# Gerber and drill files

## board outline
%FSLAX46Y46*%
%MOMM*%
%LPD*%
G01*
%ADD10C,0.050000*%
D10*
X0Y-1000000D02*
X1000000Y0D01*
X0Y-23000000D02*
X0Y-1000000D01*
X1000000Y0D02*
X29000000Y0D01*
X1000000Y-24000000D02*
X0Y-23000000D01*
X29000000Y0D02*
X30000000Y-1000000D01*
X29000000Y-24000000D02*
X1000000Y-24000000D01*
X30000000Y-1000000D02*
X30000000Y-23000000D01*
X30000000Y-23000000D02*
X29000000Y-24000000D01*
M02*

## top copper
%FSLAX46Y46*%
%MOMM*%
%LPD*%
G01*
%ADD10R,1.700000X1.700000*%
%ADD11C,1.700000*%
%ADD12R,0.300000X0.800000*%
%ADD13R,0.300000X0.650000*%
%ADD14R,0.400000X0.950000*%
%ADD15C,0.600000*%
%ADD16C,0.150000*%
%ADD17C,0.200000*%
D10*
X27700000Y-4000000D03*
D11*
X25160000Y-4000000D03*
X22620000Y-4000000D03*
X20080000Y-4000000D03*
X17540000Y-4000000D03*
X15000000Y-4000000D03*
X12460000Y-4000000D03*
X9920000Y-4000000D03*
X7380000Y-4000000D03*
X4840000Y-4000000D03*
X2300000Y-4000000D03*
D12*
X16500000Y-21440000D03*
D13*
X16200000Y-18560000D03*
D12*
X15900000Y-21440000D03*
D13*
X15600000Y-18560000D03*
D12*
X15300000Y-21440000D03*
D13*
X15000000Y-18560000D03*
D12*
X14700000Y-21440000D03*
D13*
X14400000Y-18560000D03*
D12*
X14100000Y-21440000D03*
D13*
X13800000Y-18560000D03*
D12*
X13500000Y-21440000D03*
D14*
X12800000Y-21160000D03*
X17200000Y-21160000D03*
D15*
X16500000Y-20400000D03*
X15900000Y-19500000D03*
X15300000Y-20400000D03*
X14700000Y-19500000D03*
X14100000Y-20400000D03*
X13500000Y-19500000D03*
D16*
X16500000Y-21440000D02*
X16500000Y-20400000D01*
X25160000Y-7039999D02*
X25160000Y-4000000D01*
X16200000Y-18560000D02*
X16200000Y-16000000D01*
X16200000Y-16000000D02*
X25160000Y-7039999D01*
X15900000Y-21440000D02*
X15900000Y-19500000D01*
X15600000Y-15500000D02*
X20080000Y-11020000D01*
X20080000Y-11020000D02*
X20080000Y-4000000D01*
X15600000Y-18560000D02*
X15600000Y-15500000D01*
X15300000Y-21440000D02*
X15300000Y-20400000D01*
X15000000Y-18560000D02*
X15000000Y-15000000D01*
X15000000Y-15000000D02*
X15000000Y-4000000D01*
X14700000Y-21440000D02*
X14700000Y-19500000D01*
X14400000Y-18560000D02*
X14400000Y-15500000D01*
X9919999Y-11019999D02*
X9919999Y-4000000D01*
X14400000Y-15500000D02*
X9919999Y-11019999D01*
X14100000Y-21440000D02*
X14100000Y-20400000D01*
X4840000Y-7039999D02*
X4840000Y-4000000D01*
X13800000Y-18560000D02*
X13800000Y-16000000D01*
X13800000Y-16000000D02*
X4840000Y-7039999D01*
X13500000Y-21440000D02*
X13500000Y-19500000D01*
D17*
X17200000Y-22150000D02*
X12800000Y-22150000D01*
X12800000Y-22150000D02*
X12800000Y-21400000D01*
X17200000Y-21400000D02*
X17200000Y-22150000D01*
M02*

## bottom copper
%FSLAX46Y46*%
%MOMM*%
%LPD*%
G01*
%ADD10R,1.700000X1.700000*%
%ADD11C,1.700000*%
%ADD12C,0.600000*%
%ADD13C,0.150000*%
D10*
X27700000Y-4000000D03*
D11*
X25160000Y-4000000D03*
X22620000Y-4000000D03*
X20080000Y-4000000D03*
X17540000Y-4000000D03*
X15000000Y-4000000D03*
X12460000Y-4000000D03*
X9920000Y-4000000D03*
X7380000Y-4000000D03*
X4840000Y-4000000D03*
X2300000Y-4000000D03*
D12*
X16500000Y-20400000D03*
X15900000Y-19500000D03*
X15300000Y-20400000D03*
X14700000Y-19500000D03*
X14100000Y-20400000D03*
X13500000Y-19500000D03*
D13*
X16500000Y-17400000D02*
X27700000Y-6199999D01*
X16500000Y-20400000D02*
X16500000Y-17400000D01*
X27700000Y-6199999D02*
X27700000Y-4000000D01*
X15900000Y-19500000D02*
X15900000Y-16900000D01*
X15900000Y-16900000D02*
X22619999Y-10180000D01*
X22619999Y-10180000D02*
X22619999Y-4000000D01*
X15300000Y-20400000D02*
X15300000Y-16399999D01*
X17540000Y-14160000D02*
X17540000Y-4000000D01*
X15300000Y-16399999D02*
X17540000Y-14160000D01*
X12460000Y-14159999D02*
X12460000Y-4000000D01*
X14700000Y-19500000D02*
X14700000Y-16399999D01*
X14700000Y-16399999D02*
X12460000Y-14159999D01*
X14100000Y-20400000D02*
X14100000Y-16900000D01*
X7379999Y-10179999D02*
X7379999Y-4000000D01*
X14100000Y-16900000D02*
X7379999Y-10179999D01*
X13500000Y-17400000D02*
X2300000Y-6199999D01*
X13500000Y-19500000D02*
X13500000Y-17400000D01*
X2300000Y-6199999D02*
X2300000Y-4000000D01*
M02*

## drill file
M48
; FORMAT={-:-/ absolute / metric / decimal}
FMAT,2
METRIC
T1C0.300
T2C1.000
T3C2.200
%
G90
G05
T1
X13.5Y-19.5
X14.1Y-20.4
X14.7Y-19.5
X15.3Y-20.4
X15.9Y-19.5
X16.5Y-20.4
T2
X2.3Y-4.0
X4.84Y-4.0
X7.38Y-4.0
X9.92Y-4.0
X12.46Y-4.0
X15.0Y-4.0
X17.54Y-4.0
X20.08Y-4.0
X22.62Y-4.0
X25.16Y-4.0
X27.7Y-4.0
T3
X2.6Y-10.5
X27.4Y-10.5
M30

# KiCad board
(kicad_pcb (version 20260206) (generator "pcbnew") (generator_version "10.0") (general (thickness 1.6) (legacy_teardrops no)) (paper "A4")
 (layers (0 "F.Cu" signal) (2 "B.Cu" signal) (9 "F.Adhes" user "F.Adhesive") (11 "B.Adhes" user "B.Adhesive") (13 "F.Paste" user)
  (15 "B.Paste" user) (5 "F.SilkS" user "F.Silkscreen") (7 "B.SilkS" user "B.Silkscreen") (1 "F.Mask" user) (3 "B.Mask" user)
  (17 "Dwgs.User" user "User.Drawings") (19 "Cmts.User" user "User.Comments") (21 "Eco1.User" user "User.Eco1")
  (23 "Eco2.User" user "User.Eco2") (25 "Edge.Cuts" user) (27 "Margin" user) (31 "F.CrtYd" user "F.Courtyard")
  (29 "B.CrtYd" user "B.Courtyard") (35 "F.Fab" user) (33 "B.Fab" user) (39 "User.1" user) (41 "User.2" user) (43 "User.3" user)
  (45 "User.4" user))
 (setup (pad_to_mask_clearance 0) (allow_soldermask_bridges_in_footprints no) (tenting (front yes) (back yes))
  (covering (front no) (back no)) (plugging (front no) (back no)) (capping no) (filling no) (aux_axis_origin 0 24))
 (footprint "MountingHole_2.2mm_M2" (layer "F.Cu") (at 2.6 10.5)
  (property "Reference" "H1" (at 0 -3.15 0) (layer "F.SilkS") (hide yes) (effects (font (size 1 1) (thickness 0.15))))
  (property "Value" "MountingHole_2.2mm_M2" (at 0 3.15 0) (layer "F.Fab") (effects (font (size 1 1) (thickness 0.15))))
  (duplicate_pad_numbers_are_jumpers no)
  (pad "" np_thru_hole circle (at 0 0) (size 2.2 2.2) (drill 2.2) (layers "*.Cu" "*.Mask")))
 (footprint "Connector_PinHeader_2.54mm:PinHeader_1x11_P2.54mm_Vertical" (layer "F.Cu") (at 27.7 4 -90)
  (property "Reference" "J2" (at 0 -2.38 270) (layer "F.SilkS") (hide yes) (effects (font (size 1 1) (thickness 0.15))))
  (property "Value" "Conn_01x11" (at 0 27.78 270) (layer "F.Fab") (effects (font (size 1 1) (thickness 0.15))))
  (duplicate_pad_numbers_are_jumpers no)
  (pad "1" thru_hole rect (at 0 0 270) (size 1.7 1.7) (drill 1) (layers "*.Cu" "*.Mask") (remove_unused_layers no) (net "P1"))
  (pad "2" thru_hole circle (at 0 2.54 270) (size 1.7 1.7) (drill 1) (layers "*.Cu" "*.Mask") (remove_unused_layers no) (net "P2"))
  (pad "3" thru_hole circle (at 0 5.08 270) (size 1.7 1.7) (drill 1) (layers "*.Cu" "*.Mask") (remove_unused_layers no) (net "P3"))
  (pad "4" thru_hole circle (at 0 7.62 270) (size 1.7 1.7) (drill 1) (layers "*.Cu" "*.Mask") (remove_unused_layers no) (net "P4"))
  (pad "5" thru_hole circle (at 0 10.16 270) (size 1.7 1.7) (drill 1) (layers "*.Cu" "*.Mask") (remove_unused_layers no) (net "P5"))
  (pad "6" thru_hole circle (at 0 12.7 270) (size 1.7 1.7) (drill 1) (layers "*.Cu" "*.Mask") (remove_unused_layers no) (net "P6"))
  (pad "7" thru_hole circle (at 0 15.24 270) (size 1.7 1.7) (drill 1) (layers "*.Cu" "*.Mask") (remove_unused_layers no) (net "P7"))
  (pad "8" thru_hole circle (at 0 17.78 270) (size 1.7 1.7) (drill 1) (layers "*.Cu" "*.Mask") (remove_unused_layers no) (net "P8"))
  (pad "9" thru_hole circle (at 0 20.32 270) (size 1.7 1.7) (drill 1) (layers "*.Cu" "*.Mask") (remove_unused_layers no) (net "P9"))
  (pad "10" thru_hole circle (at 0 22.86 270) (size 1.7 1.7) (drill 1) (layers "*.Cu" "*.Mask") (remove_unused_layers no) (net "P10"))
  (pad "11" thru_hole circle (at 0 25.4 270) (size 1.7 1.7) (drill 1) (layers "*.Cu" "*.Mask") (remove_unused_layers no) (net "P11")))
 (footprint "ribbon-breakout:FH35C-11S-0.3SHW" (layer "F.Cu") (at 15 20)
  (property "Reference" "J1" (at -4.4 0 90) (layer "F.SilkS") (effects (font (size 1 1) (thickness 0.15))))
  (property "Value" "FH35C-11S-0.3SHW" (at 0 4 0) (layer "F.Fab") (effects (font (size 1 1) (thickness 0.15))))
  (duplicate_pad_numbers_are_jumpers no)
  (pad "1" smd rect (at 1.5 1.44) (size 0.3 0.8) (layers "F.Cu" "F.Mask" "F.Paste") (solder_paste_margin -0.04) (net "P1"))
  (pad "2" smd rect (at 1.2 -1.44) (size 0.3 0.65) (layers "F.Cu" "F.Mask" "F.Paste") (solder_paste_margin -0.04) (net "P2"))
  (pad "3" smd rect (at 0.9 1.44) (size 0.3 0.8) (layers "F.Cu" "F.Mask" "F.Paste") (solder_paste_margin -0.04) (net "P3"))
  (pad "4" smd rect (at 0.6 -1.44) (size 0.3 0.65) (layers "F.Cu" "F.Mask" "F.Paste") (solder_paste_margin -0.04) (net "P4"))
  (pad "5" smd rect (at 0.3 1.44) (size 0.3 0.8) (layers "F.Cu" "F.Mask" "F.Paste") (solder_paste_margin -0.04) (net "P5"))
  (pad "6" smd rect (at 0 -1.44) (size 0.3 0.65) (layers "F.Cu" "F.Mask" "F.Paste") (solder_paste_margin -0.04) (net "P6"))
  (pad "7" smd rect (at -0.3 1.44) (size 0.3 0.8) (layers "F.Cu" "F.Mask" "F.Paste") (solder_paste_margin -0.04) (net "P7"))
  (pad "8" smd rect (at -0.6 -1.44) (size 0.3 0.65) (layers "F.Cu" "F.Mask" "F.Paste") (solder_paste_margin -0.04) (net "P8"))
  (pad "9" smd rect (at -0.9 1.44) (size 0.3 0.8) (layers "F.Cu" "F.Mask" "F.Paste") (solder_paste_margin -0.04) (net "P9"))
  (pad "10" smd rect (at -1.2 -1.44) (size 0.3 0.65) (layers "F.Cu" "F.Mask" "F.Paste") (solder_paste_margin -0.04) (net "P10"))
  (pad "11" smd rect (at -1.5 1.44) (size 0.3 0.8) (layers "F.Cu" "F.Mask" "F.Paste") (solder_paste_margin -0.04) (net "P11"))
  (pad "12" smd rect (at -2.2 1.16) (size 0.4 0.95) (layers "F.Cu" "F.Mask" "F.Paste") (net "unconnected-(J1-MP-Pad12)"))
  (pad "12" smd rect (at 2.2 1.16) (size 0.4 0.95) (layers "F.Cu" "F.Mask" "F.Paste") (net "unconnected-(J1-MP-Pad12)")))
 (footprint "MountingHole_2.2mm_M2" (layer "F.Cu") (at 27.4 10.5)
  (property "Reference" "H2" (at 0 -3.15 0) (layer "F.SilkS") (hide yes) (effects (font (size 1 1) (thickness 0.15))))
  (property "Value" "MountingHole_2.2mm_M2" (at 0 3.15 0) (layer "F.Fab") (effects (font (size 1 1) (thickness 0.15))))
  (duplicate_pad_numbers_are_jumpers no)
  (pad "" np_thru_hole circle (at 0 0) (size 2.2 2.2) (drill 2.2) (layers "*.Cu" "*.Mask")))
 (gr_line (start 0 1) (end 1 0) (stroke (width 0.05) (type default)) (layer "Edge.Cuts"))
 (gr_line (start 0 23) (end 0 1) (stroke (width 0.05) (type default)) (layer "Edge.Cuts"))
 (gr_line (start 1 0) (end 29 0) (stroke (width 0.05) (type default)) (layer "Edge.Cuts"))
 (gr_line (start 1 24) (end 0 23) (stroke (width 0.05) (type default)) (layer "Edge.Cuts"))
 (gr_line (start 29 0) (end 30 1) (stroke (width 0.05) (type default)) (layer "Edge.Cuts"))
 (gr_line (start 29 24) (end 1 24) (stroke (width 0.05) (type default)) (layer "Edge.Cuts"))
 (gr_line (start 30 1) (end 30 23) (stroke (width 0.05) (type default)) (layer "Edge.Cuts"))
 (gr_line (start 30 23) (end 29 24) (stroke (width 0.05) (type default)) (layer "Edge.Cuts"))
 (segment (start 16.5 21.44) (end 16.5 20.4) (width 0.15) (layer "F.Cu") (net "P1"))
 (via (at 16.5 20.4) (size 0.6) (drill 0.3) (layers "F.Cu" "B.Cu") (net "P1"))
 (segment (start 16.5 17.4) (end 27.7 6.199999) (width 0.15) (layer "B.Cu") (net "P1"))
 (segment (start 16.5 20.4) (end 16.5 17.4) (width 0.15) (layer "B.Cu") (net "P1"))
 (segment (start 27.7 6.199999) (end 27.7 4) (width 0.15) (layer "B.Cu") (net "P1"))
 (segment (start 25.16 7.039999) (end 25.16 4) (width 0.15) (layer "F.Cu") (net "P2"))
 (segment (start 16.2 18.56) (end 16.2 16) (width 0.15) (layer "F.Cu") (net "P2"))
 (segment (start 16.2 16) (end 25.16 7.039999) (width 0.15) (layer "F.Cu") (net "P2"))
 (segment (start 15.9 21.44) (end 15.9 19.5) (width 0.15) (layer "F.Cu") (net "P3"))
 (via (at 15.9 19.5) (size 0.6) (drill 0.3) (layers "F.Cu" "B.Cu") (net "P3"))
 (segment (start 15.9 19.5) (end 15.9 16.9) (width 0.15) (layer "B.Cu") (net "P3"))
 (segment (start 15.9 16.9) (end 22.619999 10.18) (width 0.15) (layer "B.Cu") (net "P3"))
 (segment (start 22.619999 10.18) (end 22.619999 4) (width 0.15) (layer "B.Cu") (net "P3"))
 (segment (start 15.6 15.5) (end 20.08 11.02) (width 0.15) (layer "F.Cu") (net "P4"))
 (segment (start 20.08 11.02) (end 20.08 4) (width 0.15) (layer "F.Cu") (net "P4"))
 (segment (start 15.6 18.56) (end 15.6 15.5) (width 0.15) (layer "F.Cu") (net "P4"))
 (segment (start 15.3 21.44) (end 15.3 20.4) (width 0.15) (layer "F.Cu") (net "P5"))
 (via (at 15.3 20.4) (size 0.6) (drill 0.3) (layers "F.Cu" "B.Cu") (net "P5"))
 (segment (start 15.3 20.4) (end 15.3 16.399999) (width 0.15) (layer "B.Cu") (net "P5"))
 (segment (start 17.54 14.16) (end 17.54 4) (width 0.15) (layer "B.Cu") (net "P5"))
 (segment (start 15.3 16.399999) (end 17.54 14.16) (width 0.15) (layer "B.Cu") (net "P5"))
 (segment (start 15 18.56) (end 15 15) (width 0.15) (layer "F.Cu") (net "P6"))
 (segment (start 15 15) (end 15 4) (width 0.15) (layer "F.Cu") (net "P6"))
 (segment (start 14.7 21.44) (end 14.7 19.5) (width 0.15) (layer "F.Cu") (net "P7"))
 (via (at 14.7 19.5) (size 0.6) (drill 0.3) (layers "F.Cu" "B.Cu") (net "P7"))
 (segment (start 12.46 14.159999) (end 12.46 4) (width 0.15) (layer "B.Cu") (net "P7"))
 (segment (start 14.7 19.5) (end 14.7 16.399999) (width 0.15) (layer "B.Cu") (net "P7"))
 (segment (start 14.7 16.399999) (end 12.46 14.159999) (width 0.15) (layer "B.Cu") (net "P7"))
 (segment (start 14.4 18.56) (end 14.4 15.5) (width 0.15) (layer "F.Cu") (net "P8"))
 (segment (start 9.919999 11.019999) (end 9.919999 4) (width 0.15) (layer "F.Cu") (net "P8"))
 (segment (start 14.4 15.5) (end 9.919999 11.019999) (width 0.15) (layer "F.Cu") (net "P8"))
 (segment (start 14.1 21.44) (end 14.1 20.4) (width 0.15) (layer "F.Cu") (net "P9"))
 (via (at 14.1 20.4) (size 0.6) (drill 0.3) (layers "F.Cu" "B.Cu") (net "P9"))
 (segment (start 14.1 20.4) (end 14.1 16.9) (width 0.15) (layer "B.Cu") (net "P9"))
 (segment (start 7.379999 10.179999) (end 7.379999 4) (width 0.15) (layer "B.Cu") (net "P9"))
 (segment (start 14.1 16.9) (end 7.379999 10.179999) (width 0.15) (layer "B.Cu") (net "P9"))
 (segment (start 4.84 7.039999) (end 4.84 4) (width 0.15) (layer "F.Cu") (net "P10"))
 (segment (start 13.8 18.56) (end 13.8 16) (width 0.15) (layer "F.Cu") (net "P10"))
 (segment (start 13.8 16) (end 4.84 7.039999) (width 0.15) (layer "F.Cu") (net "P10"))
 (segment (start 13.5 21.44) (end 13.5 19.5) (width 0.15) (layer "F.Cu") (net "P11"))
 (via (at 13.5 19.5) (size 0.6) (drill 0.3) (layers "F.Cu" "B.Cu") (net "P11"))
 (segment (start 13.5 17.4) (end 2.3 6.199999) (width 0.15) (layer "B.Cu") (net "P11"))
 (segment (start 13.5 19.5) (end 13.5 17.4) (width 0.15) (layer "B.Cu") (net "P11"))
 (segment (start 2.3 6.199999) (end 2.3 4) (width 0.15) (layer "B.Cu") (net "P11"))
 (segment (start 17.2 22.15) (end 12.8 22.15) (width 0.2) (layer "F.Cu") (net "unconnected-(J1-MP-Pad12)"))
 (segment (start 12.8 22.15) (end 12.8 21.4) (width 0.2) (layer "F.Cu") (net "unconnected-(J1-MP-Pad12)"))
 (segment (start 17.2 21.4) (end 17.2 22.15) (width 0.2) (layer "F.Cu") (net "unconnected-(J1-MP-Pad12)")))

